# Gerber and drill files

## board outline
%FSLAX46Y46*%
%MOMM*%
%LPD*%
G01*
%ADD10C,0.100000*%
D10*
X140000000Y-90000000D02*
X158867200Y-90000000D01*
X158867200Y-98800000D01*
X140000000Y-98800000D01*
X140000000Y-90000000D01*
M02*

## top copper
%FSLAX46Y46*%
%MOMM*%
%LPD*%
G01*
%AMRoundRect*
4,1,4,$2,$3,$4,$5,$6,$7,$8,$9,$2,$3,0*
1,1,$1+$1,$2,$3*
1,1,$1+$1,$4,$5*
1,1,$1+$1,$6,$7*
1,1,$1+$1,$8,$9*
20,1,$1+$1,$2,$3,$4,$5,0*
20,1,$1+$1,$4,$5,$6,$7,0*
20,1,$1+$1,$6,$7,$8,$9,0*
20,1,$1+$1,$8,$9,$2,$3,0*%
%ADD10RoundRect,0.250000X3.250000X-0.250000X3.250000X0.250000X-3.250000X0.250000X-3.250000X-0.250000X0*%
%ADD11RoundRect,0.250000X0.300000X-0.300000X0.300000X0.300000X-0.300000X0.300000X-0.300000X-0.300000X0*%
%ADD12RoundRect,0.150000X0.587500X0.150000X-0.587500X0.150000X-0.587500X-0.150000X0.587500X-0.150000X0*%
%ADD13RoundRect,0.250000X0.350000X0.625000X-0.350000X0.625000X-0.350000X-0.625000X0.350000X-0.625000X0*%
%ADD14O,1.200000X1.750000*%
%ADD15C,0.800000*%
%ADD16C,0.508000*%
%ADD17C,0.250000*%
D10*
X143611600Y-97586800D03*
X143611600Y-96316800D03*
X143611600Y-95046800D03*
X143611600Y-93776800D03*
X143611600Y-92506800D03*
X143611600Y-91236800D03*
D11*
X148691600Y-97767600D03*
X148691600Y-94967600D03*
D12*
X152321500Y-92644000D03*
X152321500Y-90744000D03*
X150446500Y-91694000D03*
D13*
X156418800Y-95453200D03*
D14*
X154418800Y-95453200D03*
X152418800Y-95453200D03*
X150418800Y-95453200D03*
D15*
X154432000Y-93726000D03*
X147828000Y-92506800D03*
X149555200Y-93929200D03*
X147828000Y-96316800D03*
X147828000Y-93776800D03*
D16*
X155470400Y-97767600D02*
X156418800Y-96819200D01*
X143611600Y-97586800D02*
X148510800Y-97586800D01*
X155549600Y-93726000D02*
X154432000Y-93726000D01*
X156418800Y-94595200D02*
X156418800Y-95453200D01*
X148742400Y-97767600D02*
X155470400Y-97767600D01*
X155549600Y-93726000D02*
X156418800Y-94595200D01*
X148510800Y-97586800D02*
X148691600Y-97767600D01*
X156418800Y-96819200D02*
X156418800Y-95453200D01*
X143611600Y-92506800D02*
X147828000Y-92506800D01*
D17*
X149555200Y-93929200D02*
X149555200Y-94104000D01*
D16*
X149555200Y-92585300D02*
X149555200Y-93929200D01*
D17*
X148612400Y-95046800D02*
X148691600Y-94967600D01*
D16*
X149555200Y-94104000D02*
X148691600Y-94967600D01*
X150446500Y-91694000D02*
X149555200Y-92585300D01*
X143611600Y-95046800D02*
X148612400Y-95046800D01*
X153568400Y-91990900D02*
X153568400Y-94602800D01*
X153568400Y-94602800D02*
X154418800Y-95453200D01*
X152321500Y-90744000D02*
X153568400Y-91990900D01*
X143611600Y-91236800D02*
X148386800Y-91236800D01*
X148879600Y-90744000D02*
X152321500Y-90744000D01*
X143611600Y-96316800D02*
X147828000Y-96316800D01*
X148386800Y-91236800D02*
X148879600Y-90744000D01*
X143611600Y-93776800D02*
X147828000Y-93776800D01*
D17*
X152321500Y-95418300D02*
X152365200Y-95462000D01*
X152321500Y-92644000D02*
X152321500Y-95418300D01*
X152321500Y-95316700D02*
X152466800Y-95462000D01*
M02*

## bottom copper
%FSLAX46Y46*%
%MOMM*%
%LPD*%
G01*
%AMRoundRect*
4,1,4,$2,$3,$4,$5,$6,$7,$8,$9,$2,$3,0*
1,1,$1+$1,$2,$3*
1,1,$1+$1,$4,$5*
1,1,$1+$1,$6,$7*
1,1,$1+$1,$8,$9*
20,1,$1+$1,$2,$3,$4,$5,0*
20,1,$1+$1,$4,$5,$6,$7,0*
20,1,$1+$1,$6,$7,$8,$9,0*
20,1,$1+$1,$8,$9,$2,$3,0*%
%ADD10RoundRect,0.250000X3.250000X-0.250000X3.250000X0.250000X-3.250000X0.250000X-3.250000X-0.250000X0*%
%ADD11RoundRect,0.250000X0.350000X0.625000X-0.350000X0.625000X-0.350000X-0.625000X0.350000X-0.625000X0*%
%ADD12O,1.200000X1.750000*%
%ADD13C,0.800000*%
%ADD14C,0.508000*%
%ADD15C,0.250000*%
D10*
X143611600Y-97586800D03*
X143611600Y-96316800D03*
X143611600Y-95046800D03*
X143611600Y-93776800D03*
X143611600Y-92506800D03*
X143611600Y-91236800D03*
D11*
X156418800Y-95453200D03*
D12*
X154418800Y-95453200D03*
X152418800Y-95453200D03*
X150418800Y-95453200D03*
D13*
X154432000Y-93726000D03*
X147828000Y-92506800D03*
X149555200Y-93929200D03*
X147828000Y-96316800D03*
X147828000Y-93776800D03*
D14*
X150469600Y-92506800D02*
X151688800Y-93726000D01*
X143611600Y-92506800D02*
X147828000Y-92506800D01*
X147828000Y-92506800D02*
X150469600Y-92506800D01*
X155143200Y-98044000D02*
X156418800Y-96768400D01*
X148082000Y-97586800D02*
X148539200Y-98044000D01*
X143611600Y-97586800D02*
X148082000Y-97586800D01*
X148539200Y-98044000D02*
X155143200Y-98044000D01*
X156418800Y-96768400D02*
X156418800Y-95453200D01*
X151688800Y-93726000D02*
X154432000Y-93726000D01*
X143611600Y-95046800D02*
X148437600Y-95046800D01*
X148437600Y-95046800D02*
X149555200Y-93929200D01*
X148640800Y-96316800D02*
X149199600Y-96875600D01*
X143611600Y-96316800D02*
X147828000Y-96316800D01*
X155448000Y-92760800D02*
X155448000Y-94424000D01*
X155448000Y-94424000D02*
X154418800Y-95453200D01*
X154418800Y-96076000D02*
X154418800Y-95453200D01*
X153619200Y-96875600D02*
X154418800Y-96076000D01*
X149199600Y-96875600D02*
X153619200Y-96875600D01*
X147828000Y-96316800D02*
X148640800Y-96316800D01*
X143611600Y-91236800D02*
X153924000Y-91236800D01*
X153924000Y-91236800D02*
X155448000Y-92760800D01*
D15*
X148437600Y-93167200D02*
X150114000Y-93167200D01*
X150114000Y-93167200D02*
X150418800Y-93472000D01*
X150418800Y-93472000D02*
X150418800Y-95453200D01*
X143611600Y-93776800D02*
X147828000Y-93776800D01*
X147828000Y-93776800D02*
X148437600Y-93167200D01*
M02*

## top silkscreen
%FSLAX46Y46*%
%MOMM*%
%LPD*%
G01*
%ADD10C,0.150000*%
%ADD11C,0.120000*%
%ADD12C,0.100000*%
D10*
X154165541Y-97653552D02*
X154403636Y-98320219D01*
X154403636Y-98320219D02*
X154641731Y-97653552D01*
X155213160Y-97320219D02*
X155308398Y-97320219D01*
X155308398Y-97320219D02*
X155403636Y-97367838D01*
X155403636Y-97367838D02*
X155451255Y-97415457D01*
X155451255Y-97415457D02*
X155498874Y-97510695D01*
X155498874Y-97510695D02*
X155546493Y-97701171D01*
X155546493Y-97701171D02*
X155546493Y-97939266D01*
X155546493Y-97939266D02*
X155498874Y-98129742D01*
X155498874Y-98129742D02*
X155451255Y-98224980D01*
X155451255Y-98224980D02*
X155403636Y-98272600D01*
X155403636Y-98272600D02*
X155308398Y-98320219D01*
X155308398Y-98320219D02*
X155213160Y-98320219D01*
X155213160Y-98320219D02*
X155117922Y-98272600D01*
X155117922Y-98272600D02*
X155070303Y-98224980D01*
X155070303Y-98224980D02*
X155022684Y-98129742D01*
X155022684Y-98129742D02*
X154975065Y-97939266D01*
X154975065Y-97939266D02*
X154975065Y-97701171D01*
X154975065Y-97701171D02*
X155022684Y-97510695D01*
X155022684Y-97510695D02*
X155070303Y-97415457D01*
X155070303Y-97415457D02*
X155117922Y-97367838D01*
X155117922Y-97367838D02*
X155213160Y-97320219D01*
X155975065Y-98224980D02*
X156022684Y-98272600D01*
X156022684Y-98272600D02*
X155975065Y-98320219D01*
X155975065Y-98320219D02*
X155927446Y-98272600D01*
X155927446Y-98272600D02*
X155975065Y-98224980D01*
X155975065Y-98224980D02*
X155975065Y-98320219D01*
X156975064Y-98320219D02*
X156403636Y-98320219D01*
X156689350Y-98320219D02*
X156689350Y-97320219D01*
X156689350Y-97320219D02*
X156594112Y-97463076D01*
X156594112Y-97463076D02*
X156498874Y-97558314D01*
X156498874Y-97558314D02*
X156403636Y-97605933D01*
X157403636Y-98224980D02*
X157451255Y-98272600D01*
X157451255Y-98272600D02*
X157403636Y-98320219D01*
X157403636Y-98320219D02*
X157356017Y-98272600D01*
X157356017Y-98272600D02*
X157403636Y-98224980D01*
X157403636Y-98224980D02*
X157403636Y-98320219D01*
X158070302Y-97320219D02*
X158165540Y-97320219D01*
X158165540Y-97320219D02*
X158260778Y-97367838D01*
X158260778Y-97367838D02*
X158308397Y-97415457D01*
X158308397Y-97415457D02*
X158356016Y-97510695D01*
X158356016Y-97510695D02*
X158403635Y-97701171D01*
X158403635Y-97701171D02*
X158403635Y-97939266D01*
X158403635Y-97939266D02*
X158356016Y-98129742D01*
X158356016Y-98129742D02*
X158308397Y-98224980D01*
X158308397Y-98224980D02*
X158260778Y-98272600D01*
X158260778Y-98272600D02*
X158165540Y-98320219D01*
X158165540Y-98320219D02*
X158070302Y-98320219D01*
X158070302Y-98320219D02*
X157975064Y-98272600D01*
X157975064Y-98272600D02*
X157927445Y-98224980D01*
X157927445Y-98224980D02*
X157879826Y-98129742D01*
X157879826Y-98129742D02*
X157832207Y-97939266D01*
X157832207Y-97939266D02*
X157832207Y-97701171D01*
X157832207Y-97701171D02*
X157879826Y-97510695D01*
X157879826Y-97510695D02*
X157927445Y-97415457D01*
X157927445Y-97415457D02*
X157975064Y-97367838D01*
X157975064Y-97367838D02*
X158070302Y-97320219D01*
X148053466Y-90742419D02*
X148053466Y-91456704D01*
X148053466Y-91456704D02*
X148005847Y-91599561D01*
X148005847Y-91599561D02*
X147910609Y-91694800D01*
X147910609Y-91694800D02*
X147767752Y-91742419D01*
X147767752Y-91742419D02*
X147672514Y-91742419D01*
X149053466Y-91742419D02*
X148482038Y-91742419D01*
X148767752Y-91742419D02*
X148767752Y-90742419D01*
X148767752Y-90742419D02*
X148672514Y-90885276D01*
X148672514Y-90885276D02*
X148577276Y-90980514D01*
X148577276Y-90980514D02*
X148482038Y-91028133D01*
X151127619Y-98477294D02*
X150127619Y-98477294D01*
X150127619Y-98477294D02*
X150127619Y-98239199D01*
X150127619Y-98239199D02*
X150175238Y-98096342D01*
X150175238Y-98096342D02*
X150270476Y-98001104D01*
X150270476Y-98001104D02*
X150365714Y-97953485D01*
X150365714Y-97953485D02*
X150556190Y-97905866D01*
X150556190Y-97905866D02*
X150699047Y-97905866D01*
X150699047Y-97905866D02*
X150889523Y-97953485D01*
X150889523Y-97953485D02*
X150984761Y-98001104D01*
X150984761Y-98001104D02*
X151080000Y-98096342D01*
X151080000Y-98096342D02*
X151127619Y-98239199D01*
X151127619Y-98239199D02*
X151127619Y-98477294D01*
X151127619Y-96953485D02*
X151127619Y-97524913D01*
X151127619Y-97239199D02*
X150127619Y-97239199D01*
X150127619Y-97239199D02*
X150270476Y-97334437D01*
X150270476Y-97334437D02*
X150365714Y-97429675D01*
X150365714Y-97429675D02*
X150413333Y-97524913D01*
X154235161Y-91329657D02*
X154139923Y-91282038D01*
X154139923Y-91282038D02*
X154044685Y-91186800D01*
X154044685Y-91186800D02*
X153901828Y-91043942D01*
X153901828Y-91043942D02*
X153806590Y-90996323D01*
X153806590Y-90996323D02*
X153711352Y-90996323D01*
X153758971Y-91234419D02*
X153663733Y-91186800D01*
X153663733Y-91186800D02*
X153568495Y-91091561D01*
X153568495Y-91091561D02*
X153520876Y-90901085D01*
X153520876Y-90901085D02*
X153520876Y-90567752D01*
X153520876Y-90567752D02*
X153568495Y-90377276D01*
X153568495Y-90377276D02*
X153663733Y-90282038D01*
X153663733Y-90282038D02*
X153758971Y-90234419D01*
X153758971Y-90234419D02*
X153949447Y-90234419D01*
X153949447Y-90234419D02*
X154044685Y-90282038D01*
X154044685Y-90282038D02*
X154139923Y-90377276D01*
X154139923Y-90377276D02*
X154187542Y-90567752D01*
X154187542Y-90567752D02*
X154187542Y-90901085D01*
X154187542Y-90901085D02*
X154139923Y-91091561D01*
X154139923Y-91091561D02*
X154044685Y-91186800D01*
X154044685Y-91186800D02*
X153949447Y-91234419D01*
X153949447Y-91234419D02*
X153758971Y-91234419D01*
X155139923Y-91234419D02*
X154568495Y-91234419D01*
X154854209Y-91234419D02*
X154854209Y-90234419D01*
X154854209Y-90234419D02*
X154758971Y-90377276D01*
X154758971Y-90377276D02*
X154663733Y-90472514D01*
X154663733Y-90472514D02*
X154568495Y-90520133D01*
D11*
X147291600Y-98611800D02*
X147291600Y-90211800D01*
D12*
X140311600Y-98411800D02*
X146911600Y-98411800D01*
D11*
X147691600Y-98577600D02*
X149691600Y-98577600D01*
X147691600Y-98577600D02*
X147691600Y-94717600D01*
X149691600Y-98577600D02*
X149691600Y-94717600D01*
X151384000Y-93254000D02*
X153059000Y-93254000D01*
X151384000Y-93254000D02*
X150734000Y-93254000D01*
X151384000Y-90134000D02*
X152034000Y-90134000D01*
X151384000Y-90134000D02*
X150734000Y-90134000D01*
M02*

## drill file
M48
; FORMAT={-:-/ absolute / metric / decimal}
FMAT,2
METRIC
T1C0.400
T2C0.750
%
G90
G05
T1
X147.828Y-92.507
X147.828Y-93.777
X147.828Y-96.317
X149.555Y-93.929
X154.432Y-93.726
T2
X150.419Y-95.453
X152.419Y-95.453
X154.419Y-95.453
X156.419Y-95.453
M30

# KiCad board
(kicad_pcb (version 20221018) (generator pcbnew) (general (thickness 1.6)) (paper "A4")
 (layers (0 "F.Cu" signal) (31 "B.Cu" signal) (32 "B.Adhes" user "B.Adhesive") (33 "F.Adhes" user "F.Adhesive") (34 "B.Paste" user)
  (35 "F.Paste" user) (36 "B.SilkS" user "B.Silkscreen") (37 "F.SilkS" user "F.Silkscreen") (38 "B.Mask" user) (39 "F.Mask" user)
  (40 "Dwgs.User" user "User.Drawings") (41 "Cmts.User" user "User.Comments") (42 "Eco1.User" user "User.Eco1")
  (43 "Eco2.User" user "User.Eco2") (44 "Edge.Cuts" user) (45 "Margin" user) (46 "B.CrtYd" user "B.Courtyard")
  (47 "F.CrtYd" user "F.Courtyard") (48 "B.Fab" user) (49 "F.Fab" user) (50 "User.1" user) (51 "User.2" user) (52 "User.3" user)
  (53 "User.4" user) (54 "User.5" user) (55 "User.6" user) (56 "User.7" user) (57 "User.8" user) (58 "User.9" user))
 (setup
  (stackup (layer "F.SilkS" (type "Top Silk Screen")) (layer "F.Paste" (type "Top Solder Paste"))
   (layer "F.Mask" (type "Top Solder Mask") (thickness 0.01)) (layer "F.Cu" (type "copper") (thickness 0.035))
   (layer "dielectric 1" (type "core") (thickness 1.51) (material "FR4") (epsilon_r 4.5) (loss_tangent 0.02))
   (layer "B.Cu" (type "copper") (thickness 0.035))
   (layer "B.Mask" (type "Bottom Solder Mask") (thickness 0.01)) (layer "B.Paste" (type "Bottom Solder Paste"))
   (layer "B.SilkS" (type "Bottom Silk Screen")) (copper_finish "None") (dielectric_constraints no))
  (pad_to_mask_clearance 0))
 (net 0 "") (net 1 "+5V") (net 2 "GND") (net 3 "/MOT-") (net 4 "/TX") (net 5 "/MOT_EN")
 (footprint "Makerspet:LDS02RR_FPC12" (layer "F.Cu") (at 143.6116 94.4118 90)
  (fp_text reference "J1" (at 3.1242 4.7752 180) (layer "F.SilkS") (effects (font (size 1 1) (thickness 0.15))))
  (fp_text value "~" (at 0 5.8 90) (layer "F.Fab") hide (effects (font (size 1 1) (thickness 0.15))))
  (fp_line (start -4.2 3.68) (end 4.2 3.68) (stroke (width 0.12) (type default)) (layer "F.SilkS"))
  (fp_line (start -4 -3.3) (end -4 3.3) (stroke (width 0.1) (type default)) (layer "F.SilkS"))
  (pad "1" smd roundrect (at -3.175 0 90) (size 1 7) (layers "F.Cu" "F.Mask") (roundrect_rratio 0.25) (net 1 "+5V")
   (thermal_bridge_angle 45))
  (pad "2" smd roundrect (at -3.175 0 90) (size 1 7) (layers "B.Cu" "B.Mask") (roundrect_rratio 0.25) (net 1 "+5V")
   (thermal_bridge_angle 45))
  (pad "3" smd roundrect (at -1.905 0 90) (size 1 7) (layers "F.Cu" "F.Mask") (roundrect_rratio 0.25) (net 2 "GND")
   (thermal_bridge_angle 45))
  (pad "4" smd roundrect (at -1.905 0 90) (size 1 7) (layers "B.Cu" "B.Mask") (roundrect_rratio 0.25) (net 2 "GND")
   (thermal_bridge_angle 45))
  (pad "5" smd roundrect (at -0.635 0 90) (size 1 7) (layers "F.Cu" "F.Mask") (roundrect_rratio 0.25) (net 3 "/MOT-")
   (thermal_bridge_angle 45))
  (pad "6" smd roundrect (at -0.635 0 90) (size 1 7) (layers "B.Cu" "B.Mask") (roundrect_rratio 0.25) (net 3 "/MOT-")
   (thermal_bridge_angle 45))
  (pad "7" smd roundrect (at 0.635 0 90) (size 1 7) (layers "F.Cu" "F.Mask") (roundrect_rratio 0.25) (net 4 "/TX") (thermal_bridge_angle 45))
  (pad "8" smd roundrect (at 0.635 0 90) (size 1 7) (layers "B.Cu" "B.Mask") (roundrect_rratio 0.25) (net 4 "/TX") (thermal_bridge_angle 45))
  (pad "9" smd roundrect (at 1.905 0 90) (size 1 7) (layers "F.Cu" "F.Mask") (roundrect_rratio 0.25) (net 1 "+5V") (thermal_bridge_angle 45))
  (pad "10" smd roundrect (at 1.905 0 90) (size 1 7) (layers "B.Cu" "B.Mask") (roundrect_rratio 0.25) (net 1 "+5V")
   (thermal_bridge_angle 45))
  (pad "11" smd roundrect (at 3.175 0 90) (size 1 7) (layers "F.Cu" "F.Mask") (roundrect_rratio 0.25) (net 2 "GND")
   (thermal_bridge_angle 45))
  (pad "12" smd roundrect (at 3.175 0 90) (size 1 7) (layers "B.Cu" "B.Mask") (roundrect_rratio 0.25) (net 2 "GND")
   (thermal_bridge_angle 45)))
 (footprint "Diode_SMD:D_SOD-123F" (layer "F.Cu") (at 148.6916 96.3676 90)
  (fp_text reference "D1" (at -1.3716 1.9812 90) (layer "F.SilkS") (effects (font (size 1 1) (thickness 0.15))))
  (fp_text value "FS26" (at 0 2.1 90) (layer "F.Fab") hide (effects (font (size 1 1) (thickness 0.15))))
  (fp_line (start -2.21 -1) (end -2.21 1) (stroke (width 0.12) (type solid)) (layer "F.SilkS"))
  (fp_line (start -2.21 -1) (end 1.65 -1) (stroke (width 0.12) (type solid)) (layer "F.SilkS"))
  (fp_line (start -2.21 1) (end 1.65 1) (stroke (width 0.12) (type solid)) (layer "F.SilkS"))
  (pad "1" smd roundrect (at -1.4 0 90) (size 1.1 1.1) (layers "F.Cu" "F.Paste" "F.Mask") (roundrect_rratio 0.2272727273) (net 1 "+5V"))
  (pad "2" smd roundrect (at 1.4 0 90) (size 1.1 1.1) (layers "F.Cu" "F.Paste" "F.Mask") (roundrect_rratio 0.2272727273) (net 3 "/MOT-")))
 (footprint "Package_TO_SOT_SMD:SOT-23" (layer "F.Cu") (at 151.384 91.694 180)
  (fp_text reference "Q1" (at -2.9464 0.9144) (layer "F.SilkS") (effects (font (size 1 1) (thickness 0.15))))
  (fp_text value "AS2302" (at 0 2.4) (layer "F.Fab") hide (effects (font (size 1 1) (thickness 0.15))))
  (fp_line (start 0 -1.56) (end -1.675 -1.56) (stroke (width 0.12) (type solid)) (layer "F.SilkS"))
  (fp_line (start 0 -1.56) (end 0.65 -1.56) (stroke (width 0.12) (type solid)) (layer "F.SilkS"))
  (fp_line (start 0 1.56) (end -0.65 1.56) (stroke (width 0.12) (type solid)) (layer "F.SilkS"))
  (fp_line (start 0 1.56) (end 0.65 1.56) (stroke (width 0.12) (type solid)) (layer "F.SilkS"))
  (pad "1" smd roundrect (at -0.9375 -0.95 180) (size 1.475 0.6) (layers "F.Cu" "F.Paste" "F.Mask") (roundrect_rratio 0.25)
   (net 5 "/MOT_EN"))
  (pad "2" smd roundrect (at -0.9375 0.95 180) (size 1.475 0.6) (layers "F.Cu" "F.Paste" "F.Mask") (roundrect_rratio 0.25) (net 2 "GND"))
  (pad "3" smd roundrect (at 0.9375 0 180) (size 1.475 0.6) (layers "F.Cu" "F.Paste" "F.Mask") (roundrect_rratio 0.25) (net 3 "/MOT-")))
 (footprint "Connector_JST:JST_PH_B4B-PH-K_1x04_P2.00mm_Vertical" (layer "B.Cu") (at 156.4188 95.4532 180)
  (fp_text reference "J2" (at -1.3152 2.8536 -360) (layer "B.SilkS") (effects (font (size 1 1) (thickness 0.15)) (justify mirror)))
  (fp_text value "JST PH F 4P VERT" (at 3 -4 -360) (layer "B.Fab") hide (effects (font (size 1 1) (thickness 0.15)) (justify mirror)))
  (pad "1" thru_hole roundrect (at 0 0 180) (size 1.2 1.75) (drill 0.75) (layers "*.Cu" "*.Mask") (roundrect_rratio 0.2083333333)
   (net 1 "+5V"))
  (pad "2" thru_hole oval (at 2 0 180) (size 1.2 1.75) (drill 0.75) (layers "*.Cu" "*.Mask") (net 2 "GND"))
  (pad "3" thru_hole oval (at 4 0 180) (size 1.2 1.75) (drill 0.75) (layers "*.Cu" "*.Mask") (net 5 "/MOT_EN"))
  (pad "4" thru_hole oval (at 6 0 180) (size 1.2 1.75) (drill 0.75) (layers "*.Cu" "*.Mask") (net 4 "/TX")))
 (gr_rect (start 140 90) (end 158.8672 98.8) (stroke (width 0.1) (type default)) (fill none) (layer "Edge.Cuts"))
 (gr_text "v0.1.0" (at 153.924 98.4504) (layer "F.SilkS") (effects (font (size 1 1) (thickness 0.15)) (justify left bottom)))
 (segment (start 155.4704 97.7676) (end 156.4188 96.8192) (width 0.508) (layer "F.Cu") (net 1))
 (segment (start 143.6116 97.5868) (end 148.5108 97.5868) (width 0.508) (layer "F.Cu") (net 1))
 (segment (start 155.5496 93.726) (end 154.432 93.726) (width 0.508) (layer "F.Cu") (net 1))
 (segment (start 156.4188 94.5952) (end 156.4188 95.4532) (width 0.508) (layer "F.Cu") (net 1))
 (segment (start 148.7424 97.7676) (end 155.4704 97.7676) (width 0.508) (layer "F.Cu") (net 1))
 (segment (start 155.5496 93.726) (end 156.4188 94.5952) (width 0.508) (layer "F.Cu") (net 1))
 (segment (start 148.5108 97.5868) (end 148.6916 97.7676) (width 0.508) (layer "F.Cu") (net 1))
 (segment (start 156.4188 96.8192) (end 156.4188 95.4532) (width 0.508) (layer "F.Cu") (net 1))
 (segment (start 143.6116 92.5068) (end 147.828 92.5068) (width 0.508) (layer "F.Cu") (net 1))
 (via (at 154.432 93.726) (size 0.8) (drill 0.4) (layers "F.Cu" "B.Cu") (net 1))
 (via (at 147.828 92.5068) (size 0.8) (drill 0.4) (layers "F.Cu" "B.Cu") (free) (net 1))
 (segment (start 150.4696 92.5068) (end 151.6888 93.726) (width 0.508) (layer "B.Cu") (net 1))
 (segment (start 143.6116 92.5068) (end 147.828 92.5068) (width 0.508) (layer "B.Cu") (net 1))
 (segment (start 147.828 92.5068) (end 150.4696 92.5068) (width 0.508) (layer "B.Cu") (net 1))
 (segment (start 155.1432 98.044) (end 156.4188 96.7684) (width 0.508) (layer "B.Cu") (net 1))
 (segment (start 148.082 97.5868) (end 148.5392 98.044) (width 0.508) (layer "B.Cu") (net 1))
 (segment (start 143.6116 97.5868) (end 148.082 97.5868) (width 0.508) (layer "B.Cu") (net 1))
 (segment (start 148.5392 98.044) (end 155.1432 98.044) (width 0.508) (layer "B.Cu") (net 1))
 (segment (start 156.4188 96.7684) (end 156.4188 95.4532) (width 0.508) (layer "B.Cu") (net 1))
 (segment (start 151.6888 93.726) (end 154.432 93.726) (width 0.508) (layer "B.Cu") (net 1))
 (segment (start 149.5552 93.9292) (end 149.5552 94.104) (width 0.25) (layer "F.Cu") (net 3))
 (segment (start 149.5552 92.5853) (end 149.5552 93.9292) (width 0.508) (layer "F.Cu") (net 3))
 (segment (start 148.6124 95.0468) (end 148.6916 94.9676) (width 0.25) (layer "F.Cu") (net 3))
 (segment (start 149.5552 94.104) (end 148.6916 94.9676) (width 0.508) (layer "F.Cu") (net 3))
 (segment (start 150.4465 91.694) (end 149.5552 92.5853) (width 0.508) (layer "F.Cu") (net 3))
 (segment (start 143.6116 95.0468) (end 148.6124 95.0468) (width 0.508) (layer "F.Cu") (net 3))
 (via (at 149.5552 93.9292) (size 0.8) (drill 0.4) (layers "F.Cu" "B.Cu") (free) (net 3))
 (segment (start 143.6116 95.0468) (end 148.4376 95.0468) (width 0.508) (layer "B.Cu") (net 3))
 (segment (start 148.4376 95.0468) (end 149.5552 93.9292) (width 0.508) (layer "B.Cu") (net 3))
 (segment (start 153.5684 91.9909) (end 153.5684 94.6028) (width 0.508) (layer "F.Cu") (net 2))
 (segment (start 153.5684 94.6028) (end 154.4188 95.4532) (width 0.508) (layer "F.Cu") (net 2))
 (segment (start 152.3215 90.744) (end 153.5684 91.9909) (width 0.508) (layer "F.Cu") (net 2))
 (segment (start 143.6116 91.2368) (end 148.3868 91.2368) (width 0.508) (layer "F.Cu") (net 2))
 (segment (start 148.8796 90.744) (end 152.3215 90.744) (width 0.508) (layer "F.Cu") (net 2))
 (segment (start 143.6116 96.3168) (end 147.828 96.3168) (width 0.508) (layer "F.Cu") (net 2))
 (segment (start 148.3868 91.2368) (end 148.8796 90.744) (width 0.508) (layer "F.Cu") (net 2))
 (via (at 147.828 96.3168) (size 0.8) (drill 0.4) (layers "F.Cu" "B.Cu") (free) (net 2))
 (segment (start 148.6408 96.3168) (end 149.1996 96.8756) (width 0.508) (layer "B.Cu") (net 2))
 (segment (start 143.6116 96.3168) (end 147.828 96.3168) (width 0.508) (layer "B.Cu") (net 2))
 (segment (start 155.448 92.7608) (end 155.448 94.424) (width 0.508) (layer "B.Cu") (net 2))
 (segment (start 155.448 94.424) (end 154.4188 95.4532) (width 0.508) (layer "B.Cu") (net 2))
 (segment (start 154.4188 96.076) (end 154.4188 95.4532) (width 0.508) (layer "B.Cu") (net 2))
 (segment (start 153.6192 96.8756) (end 154.4188 96.076) (width 0.508) (layer "B.Cu") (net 2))
 (segment (start 149.1996 96.8756) (end 153.6192 96.8756) (width 0.508) (layer "B.Cu") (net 2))
 (segment (start 147.828 96.3168) (end 148.6408 96.3168) (width 0.508) (layer "B.Cu") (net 2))
 (segment (start 143.6116 91.2368) (end 153.924 91.2368) (width 0.508) (layer "B.Cu") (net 2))
 (segment (start 153.924 91.2368) (end 155.448 92.7608) (width 0.508) (layer "B.Cu") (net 2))
 (segment (start 143.6116 93.7768) (end 147.828 93.7768) (width 0.508) (layer "F.Cu") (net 4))
 (via (at 147.828 93.7768) (size 0.8) (drill 0.4) (layers "F.Cu" "B.Cu") (free) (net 4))
 (segment (start 148.4376 93.1672) (end 150.114 93.1672) (width 0.25) (layer "B.Cu") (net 4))
 (segment (start 150.114 93.1672) (end 150.4188 93.472) (width 0.25) (layer "B.Cu") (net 4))
 (segment (start 150.4188 93.472) (end 150.4188 95.4532) (width 0.25) (layer "B.Cu") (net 4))
 (segment (start 143.6116 93.7768) (end 147.828 93.7768) (width 0.25) (layer "B.Cu") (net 4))
 (segment (start 147.828 93.7768) (end 148.4376 93.1672) (width 0.25) (layer "B.Cu") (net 4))
 (segment (start 152.3215 95.4183) (end 152.3652 95.462) (width 0.25) (layer "F.Cu") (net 5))
 (segment (start 152.3215 92.644) (end 152.3215 95.4183) (width 0.25) (layer "F.Cu") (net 5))
 (segment (start 152.3215 95.3167) (end 152.4668 95.462) (width 0.25) (layer "F.Cu") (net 5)))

